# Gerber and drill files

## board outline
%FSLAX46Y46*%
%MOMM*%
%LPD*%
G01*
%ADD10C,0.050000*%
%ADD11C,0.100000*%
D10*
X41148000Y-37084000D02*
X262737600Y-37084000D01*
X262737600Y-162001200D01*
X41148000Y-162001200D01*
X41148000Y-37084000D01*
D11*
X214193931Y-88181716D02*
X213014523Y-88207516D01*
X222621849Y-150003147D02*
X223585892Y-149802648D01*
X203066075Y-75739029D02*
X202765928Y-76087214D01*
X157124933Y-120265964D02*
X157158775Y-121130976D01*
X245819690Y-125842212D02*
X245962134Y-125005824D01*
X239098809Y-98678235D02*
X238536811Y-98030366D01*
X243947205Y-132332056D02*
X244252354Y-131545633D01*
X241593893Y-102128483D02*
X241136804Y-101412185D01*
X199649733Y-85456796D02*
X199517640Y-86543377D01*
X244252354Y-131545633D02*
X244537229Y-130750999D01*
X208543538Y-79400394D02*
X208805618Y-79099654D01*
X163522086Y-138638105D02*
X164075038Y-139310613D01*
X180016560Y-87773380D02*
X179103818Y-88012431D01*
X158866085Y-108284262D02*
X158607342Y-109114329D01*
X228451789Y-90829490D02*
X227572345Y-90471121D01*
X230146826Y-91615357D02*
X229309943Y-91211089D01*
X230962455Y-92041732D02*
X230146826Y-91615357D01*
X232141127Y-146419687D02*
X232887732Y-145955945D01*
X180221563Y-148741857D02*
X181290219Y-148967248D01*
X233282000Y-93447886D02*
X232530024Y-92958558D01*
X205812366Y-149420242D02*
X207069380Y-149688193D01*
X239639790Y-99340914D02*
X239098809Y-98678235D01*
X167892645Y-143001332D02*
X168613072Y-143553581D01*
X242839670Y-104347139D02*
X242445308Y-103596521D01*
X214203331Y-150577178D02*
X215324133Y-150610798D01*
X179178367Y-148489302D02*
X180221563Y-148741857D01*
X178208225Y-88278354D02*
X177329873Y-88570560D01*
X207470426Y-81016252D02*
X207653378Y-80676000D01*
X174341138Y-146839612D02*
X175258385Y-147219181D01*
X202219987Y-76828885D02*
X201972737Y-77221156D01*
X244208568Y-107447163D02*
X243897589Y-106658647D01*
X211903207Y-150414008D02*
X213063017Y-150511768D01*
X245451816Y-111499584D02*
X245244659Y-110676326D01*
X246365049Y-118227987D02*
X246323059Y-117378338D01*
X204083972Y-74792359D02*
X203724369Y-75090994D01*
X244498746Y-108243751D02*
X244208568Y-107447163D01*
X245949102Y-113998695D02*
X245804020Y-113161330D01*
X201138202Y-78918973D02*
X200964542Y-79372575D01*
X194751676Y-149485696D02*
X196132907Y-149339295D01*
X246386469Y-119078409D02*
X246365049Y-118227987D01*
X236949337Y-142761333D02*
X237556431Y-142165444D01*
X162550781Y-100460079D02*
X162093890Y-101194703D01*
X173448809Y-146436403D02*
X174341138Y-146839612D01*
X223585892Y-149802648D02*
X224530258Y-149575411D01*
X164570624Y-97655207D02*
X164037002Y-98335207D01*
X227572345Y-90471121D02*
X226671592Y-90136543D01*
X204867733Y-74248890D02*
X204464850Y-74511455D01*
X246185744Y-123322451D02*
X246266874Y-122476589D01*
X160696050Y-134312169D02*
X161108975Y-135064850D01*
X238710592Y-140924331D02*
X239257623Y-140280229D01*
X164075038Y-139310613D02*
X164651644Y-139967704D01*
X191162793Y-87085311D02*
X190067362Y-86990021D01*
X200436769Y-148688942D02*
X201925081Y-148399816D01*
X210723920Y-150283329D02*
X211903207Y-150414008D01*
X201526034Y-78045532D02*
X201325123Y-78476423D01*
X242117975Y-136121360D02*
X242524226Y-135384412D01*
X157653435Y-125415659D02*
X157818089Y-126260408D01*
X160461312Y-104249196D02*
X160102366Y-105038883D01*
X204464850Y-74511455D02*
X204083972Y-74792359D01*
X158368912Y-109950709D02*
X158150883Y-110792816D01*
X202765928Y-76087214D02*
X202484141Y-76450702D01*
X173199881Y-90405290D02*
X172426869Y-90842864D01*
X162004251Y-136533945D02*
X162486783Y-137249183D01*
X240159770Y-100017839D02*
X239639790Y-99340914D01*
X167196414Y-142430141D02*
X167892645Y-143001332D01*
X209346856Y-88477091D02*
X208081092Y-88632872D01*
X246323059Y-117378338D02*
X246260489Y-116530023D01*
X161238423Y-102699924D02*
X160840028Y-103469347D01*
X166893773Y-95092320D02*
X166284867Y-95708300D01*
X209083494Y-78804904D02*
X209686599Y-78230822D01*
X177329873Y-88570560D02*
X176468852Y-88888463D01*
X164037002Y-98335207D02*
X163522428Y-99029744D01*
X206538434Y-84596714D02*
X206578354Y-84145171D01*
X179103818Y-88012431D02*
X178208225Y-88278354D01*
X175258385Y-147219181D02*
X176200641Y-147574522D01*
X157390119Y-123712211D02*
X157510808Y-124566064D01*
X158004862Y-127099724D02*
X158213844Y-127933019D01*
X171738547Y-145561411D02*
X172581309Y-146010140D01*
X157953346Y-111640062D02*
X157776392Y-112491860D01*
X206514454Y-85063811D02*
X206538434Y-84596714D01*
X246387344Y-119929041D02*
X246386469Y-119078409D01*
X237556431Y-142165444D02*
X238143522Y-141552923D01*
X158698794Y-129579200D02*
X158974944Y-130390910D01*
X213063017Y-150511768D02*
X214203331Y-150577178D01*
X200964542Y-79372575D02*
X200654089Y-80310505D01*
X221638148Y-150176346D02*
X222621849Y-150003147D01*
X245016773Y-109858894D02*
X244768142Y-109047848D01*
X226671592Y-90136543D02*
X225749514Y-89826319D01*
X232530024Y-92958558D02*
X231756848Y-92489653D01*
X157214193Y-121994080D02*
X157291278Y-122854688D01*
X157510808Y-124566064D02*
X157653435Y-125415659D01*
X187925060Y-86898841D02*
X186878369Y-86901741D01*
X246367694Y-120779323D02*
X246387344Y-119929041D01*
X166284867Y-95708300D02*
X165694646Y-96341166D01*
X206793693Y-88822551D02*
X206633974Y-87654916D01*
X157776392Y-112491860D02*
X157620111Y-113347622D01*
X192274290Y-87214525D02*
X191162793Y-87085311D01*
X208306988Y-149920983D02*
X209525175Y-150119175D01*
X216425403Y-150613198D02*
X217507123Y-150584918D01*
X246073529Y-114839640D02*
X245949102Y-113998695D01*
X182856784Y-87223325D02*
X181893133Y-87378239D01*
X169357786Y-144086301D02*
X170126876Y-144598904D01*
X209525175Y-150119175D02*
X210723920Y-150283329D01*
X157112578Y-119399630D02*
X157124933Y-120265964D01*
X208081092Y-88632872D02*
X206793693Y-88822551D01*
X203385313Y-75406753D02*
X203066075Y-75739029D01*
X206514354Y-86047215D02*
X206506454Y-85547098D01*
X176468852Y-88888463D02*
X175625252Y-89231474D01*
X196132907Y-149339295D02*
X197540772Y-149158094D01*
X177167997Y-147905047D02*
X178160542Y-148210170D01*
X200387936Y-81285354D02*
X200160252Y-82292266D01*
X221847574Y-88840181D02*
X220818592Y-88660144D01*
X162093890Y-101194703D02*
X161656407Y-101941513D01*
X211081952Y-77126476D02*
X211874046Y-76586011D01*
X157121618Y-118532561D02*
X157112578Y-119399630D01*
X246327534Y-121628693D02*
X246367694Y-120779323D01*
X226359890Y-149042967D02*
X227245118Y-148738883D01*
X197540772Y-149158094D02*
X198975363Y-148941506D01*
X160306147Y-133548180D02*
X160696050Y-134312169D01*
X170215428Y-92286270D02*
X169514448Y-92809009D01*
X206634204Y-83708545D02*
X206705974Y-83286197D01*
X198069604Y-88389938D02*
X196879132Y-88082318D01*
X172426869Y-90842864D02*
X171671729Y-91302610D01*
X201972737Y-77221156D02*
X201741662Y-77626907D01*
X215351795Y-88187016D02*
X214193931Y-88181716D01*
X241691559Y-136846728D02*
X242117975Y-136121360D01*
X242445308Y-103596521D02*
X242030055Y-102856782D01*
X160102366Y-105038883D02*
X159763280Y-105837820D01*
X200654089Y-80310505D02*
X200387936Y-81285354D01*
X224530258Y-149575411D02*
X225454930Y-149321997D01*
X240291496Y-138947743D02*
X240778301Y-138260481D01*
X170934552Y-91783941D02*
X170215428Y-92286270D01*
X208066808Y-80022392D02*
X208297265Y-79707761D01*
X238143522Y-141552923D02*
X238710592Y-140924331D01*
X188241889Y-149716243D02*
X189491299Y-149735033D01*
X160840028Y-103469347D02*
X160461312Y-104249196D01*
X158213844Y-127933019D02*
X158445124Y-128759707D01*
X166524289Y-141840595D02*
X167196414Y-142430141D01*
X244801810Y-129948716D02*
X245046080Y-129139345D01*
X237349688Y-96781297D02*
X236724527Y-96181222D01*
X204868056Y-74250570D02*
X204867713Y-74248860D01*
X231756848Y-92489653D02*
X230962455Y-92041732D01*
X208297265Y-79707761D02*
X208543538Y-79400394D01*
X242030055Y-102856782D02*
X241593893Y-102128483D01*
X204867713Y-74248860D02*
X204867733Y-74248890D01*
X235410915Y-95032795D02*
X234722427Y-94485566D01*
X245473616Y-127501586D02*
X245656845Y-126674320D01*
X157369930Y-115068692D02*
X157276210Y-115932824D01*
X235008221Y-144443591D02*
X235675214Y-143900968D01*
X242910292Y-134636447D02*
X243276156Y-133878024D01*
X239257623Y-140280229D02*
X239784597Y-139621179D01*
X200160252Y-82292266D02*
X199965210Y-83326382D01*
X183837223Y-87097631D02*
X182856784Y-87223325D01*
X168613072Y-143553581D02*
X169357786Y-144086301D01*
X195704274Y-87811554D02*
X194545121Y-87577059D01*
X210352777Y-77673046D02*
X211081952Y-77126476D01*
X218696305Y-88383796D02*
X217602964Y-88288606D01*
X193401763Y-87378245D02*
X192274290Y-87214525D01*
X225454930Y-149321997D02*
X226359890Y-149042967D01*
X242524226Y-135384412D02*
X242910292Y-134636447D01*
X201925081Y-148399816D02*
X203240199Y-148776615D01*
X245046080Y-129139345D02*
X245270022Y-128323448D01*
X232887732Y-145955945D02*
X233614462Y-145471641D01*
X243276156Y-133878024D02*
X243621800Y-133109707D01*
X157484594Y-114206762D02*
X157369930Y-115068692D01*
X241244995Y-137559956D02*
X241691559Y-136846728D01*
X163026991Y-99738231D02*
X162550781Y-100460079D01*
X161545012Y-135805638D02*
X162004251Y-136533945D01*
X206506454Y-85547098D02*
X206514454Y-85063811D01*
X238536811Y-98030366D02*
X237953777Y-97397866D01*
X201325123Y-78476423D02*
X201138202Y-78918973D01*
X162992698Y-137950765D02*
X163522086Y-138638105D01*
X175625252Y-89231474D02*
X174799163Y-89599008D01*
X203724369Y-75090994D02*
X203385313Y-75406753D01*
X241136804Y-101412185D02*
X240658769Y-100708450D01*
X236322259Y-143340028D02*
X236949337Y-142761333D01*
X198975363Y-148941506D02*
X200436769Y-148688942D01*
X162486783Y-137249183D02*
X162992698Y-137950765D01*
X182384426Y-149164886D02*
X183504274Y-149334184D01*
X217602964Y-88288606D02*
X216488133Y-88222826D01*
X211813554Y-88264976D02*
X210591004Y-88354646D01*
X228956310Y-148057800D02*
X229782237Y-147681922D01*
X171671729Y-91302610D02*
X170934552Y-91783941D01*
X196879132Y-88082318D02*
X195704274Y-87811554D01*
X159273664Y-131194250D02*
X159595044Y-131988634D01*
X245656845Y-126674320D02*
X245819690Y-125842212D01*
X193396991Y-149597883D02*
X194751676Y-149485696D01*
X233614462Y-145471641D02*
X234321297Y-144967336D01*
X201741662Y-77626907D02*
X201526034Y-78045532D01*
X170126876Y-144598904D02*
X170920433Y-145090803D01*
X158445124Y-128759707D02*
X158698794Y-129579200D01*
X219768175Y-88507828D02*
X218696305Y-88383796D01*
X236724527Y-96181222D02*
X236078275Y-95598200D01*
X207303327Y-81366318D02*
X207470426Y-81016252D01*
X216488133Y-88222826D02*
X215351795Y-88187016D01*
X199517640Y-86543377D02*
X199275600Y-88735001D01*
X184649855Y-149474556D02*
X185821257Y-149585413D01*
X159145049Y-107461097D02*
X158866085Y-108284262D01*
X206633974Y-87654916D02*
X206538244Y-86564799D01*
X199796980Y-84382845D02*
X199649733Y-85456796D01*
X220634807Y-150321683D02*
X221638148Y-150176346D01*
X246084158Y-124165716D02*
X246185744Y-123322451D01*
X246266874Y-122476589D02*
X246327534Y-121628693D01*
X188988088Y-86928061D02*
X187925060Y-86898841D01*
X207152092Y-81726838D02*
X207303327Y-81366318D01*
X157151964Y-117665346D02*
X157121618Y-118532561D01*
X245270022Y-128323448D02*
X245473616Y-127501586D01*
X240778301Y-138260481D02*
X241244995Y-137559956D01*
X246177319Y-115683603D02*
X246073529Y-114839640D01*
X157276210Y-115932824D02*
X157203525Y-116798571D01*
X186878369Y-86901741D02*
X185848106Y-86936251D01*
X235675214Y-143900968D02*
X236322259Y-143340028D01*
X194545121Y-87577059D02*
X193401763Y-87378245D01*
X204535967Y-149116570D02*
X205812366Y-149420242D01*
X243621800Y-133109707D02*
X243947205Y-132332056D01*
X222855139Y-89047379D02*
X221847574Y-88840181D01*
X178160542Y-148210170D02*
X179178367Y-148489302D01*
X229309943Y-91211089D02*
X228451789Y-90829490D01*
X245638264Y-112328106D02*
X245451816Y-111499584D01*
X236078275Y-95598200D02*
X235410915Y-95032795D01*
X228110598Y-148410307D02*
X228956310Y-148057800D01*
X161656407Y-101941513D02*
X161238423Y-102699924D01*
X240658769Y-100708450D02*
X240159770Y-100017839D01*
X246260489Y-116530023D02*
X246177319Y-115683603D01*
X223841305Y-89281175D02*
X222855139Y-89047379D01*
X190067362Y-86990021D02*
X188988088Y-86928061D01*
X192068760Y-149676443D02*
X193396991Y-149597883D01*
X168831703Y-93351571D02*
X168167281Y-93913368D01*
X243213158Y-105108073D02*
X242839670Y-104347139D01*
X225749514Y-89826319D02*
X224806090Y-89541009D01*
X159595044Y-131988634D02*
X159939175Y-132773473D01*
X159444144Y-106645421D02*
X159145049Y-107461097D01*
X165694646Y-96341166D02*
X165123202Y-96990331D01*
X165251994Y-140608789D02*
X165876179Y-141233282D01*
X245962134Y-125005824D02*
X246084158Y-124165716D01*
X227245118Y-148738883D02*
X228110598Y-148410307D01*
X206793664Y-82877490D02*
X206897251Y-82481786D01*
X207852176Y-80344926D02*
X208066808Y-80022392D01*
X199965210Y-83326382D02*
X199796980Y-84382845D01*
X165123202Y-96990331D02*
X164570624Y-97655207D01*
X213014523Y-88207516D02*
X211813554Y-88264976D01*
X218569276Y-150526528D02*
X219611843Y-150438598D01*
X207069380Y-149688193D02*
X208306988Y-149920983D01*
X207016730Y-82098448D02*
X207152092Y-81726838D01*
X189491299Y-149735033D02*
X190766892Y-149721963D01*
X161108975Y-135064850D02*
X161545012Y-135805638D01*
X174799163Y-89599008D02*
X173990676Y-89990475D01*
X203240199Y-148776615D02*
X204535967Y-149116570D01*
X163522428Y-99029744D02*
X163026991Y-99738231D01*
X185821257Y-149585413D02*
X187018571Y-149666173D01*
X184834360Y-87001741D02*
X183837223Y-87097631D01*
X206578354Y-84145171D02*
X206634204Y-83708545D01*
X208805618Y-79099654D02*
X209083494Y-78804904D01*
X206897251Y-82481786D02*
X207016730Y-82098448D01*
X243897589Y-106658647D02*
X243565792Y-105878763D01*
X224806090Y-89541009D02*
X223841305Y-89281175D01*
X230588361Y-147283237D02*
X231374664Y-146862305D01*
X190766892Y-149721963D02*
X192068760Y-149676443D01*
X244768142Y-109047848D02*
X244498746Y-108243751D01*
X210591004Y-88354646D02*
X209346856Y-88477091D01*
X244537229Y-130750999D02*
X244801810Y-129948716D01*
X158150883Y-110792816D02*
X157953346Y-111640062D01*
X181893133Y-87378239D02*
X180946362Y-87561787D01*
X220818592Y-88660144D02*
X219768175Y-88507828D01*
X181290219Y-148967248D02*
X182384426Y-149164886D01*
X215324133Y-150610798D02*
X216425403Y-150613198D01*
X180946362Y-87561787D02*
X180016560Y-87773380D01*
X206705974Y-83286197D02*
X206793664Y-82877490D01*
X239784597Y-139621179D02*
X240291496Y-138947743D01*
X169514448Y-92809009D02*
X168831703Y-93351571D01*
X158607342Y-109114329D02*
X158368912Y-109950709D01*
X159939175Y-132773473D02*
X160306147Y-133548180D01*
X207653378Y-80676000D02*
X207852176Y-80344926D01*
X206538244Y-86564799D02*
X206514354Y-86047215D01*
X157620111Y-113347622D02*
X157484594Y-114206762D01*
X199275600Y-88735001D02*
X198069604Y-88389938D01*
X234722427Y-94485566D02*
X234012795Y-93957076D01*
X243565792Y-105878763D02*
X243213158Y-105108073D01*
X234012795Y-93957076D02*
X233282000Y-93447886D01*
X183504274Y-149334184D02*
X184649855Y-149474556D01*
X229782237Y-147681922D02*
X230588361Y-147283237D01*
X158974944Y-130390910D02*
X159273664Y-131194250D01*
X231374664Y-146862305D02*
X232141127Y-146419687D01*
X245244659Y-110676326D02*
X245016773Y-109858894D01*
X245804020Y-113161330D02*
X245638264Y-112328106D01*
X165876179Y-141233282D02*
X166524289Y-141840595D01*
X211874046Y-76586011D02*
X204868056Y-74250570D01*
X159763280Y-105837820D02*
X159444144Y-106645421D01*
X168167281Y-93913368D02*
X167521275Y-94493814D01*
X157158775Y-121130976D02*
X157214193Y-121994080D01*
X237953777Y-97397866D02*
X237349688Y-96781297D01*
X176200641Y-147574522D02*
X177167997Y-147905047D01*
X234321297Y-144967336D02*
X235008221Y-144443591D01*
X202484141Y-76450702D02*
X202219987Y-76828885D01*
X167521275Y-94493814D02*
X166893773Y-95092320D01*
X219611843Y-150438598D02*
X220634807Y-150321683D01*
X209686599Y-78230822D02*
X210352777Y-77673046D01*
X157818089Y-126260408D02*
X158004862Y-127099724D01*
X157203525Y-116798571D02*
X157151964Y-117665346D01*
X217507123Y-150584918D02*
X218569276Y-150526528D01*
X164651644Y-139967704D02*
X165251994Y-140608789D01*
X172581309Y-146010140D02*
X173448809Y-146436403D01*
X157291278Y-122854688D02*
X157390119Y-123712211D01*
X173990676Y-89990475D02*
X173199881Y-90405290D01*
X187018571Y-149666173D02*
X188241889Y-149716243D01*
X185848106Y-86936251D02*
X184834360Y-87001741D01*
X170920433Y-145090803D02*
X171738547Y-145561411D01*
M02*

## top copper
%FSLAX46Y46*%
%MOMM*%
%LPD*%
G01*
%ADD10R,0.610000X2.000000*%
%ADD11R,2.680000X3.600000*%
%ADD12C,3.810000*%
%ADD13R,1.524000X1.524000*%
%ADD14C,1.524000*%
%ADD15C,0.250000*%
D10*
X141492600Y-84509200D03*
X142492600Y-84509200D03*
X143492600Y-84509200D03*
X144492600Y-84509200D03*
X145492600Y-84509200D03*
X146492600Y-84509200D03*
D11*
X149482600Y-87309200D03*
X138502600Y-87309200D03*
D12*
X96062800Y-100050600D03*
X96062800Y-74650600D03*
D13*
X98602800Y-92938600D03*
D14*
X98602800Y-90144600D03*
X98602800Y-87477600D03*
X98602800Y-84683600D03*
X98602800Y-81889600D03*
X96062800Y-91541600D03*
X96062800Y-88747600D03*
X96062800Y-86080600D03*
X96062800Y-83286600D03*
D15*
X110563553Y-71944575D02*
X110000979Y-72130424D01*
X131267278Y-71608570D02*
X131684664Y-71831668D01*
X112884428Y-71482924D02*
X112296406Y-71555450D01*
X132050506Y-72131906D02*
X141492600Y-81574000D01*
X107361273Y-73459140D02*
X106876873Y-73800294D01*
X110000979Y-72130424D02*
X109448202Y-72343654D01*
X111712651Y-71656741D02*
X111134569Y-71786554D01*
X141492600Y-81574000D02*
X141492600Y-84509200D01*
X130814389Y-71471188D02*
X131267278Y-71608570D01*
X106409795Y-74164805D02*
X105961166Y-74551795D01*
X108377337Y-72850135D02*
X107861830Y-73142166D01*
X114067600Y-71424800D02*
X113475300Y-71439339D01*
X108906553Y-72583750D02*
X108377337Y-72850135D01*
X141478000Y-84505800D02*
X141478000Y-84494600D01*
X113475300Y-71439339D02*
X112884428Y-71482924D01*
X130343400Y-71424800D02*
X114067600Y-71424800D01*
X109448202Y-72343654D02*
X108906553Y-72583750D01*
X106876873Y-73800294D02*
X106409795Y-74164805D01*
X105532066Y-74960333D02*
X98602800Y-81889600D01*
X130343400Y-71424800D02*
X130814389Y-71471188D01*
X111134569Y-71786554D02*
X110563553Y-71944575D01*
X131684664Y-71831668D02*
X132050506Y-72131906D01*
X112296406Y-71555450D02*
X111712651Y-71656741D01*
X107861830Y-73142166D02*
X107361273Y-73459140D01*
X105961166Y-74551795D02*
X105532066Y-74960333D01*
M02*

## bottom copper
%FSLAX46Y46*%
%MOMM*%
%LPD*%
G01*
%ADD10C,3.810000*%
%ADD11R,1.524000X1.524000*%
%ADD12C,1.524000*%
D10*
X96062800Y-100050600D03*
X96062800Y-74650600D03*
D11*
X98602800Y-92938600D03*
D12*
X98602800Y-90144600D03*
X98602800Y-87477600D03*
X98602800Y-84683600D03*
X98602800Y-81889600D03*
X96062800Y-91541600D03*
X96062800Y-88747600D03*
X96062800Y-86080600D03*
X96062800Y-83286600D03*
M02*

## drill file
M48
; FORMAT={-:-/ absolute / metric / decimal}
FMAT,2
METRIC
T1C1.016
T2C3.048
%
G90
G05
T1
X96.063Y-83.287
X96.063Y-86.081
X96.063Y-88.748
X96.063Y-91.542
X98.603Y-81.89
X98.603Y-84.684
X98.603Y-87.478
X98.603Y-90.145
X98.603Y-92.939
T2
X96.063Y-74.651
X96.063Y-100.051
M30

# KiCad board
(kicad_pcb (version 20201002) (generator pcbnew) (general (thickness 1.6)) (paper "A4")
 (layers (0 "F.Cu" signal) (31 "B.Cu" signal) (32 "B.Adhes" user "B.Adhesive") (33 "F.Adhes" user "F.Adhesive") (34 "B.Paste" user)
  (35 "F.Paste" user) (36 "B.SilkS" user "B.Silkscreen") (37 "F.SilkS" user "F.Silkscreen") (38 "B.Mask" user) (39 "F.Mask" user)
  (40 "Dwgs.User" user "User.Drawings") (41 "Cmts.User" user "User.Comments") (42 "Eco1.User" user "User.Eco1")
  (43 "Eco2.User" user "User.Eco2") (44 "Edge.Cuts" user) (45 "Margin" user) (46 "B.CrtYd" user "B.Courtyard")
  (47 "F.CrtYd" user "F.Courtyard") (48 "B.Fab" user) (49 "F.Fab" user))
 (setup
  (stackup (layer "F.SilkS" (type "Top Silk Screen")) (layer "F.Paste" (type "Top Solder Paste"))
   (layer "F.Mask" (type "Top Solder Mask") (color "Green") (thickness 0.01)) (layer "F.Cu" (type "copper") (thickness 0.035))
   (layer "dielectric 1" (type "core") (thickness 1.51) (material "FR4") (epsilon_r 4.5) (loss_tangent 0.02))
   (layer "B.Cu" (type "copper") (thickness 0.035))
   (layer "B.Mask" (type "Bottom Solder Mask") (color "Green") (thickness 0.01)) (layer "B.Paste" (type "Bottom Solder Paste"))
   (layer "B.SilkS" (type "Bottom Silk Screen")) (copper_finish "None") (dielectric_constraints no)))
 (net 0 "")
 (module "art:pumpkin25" (layer "F.Cu") (at 201.0156 117.475)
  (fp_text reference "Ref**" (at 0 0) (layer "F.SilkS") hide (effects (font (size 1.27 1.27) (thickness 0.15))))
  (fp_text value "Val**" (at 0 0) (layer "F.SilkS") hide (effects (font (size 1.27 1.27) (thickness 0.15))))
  (fp_line (start 13.178331 -29.293284) (end 11.998923 -29.267484) (layer "Edge.Cuts") (width 0.1))
  (fp_line (start 21.606249 32.528147) (end 22.570292 32.327648) (layer "Edge.Cuts") (width 0.1))
  (fp_line (start 2.050475 -41.735971) (end 1.750328 -41.387786) (layer "Edge.Cuts") (width 0.1))
  (fp_line (start -43.890667 2.790964) (end -43.856825 3.655976) (layer "Edge.Cuts") (width 0.1))
  (fp_line (start 44.80409 8.367212) (end 44.946534 7.530824) (layer "Edge.Cuts") (width 0.1))
  (fp_line (start 38.083209 -18.796765) (end 37.521211 -19.444634) (layer "Edge.Cuts") (width 0.1))
  (fp_line (start 42.931605 14.857056) (end 43.236754 14.070633) (layer "Edge.Cuts") (width 0.1))
  (fp_line (start 40.578293 -15.346517) (end 40.121204 -16.062815) (layer "Edge.Cuts") (width 0.1))
  (fp_line (start -1.365867 -32.018204) (end -1.49796 -30.931623) (layer "Edge.Cuts") (width 0.1))
  (fp_line (start 43.236754 14.070633) (end 43.521629 13.275999) (layer "Edge.Cuts") (width 0.1))
  (fp_line (start 7.527938 -38.074606) (end 7.790018 -38.375346) (layer "Edge.Cuts") (width 0.1))
  (fp_line (start -37.493514 21.163105) (end -36.940562 21.835613) (layer "Edge.Cuts") (width 0.1))
  (fp_line (start -20.99904 -29.70162) (end -21.911782 -29.462569) (layer "Edge.Cuts") (width 0.1))
  (fp_line (start -42.149515 -9.190738) (end -42.408258 -8.360671) (layer "Edge.Cuts") (width 0.1))
  (fp_line (start 27.436189 -26.64551) (end 26.556745 -27.003879) (layer "Edge.Cuts") (width 0.1))
  (fp_line (start 29.131226 -25.859643) (end 28.294343 -26.263911) (layer "Edge.Cuts") (width 0.1))
  (fp_line (start 29.946855 -25.433268) (end 29.131226 -25.859643) (layer "Edge.Cuts") (width 0.1))
  (fp_line (start 31.125527 28.944687) (end 31.872132 28.480945) (layer "Edge.Cuts") (width 0.1))
  (fp_line (start -20.794037 31.266857) (end -19.725381 31.492248) (layer "Edge.Cuts") (width 0.1))
  (fp_line (start 32.2664 -24.027114) (end 31.514424 -24.516442) (layer "Edge.Cuts") (width 0.1))
  (fp_line (start 4.796766 31.945242) (end 6.05378 32.213193) (layer "Edge.Cuts") (width 0.1))
  (fp_line (start 38.62419 -18.134086) (end 38.083209 -18.796765) (layer "Edge.Cuts") (width 0.1))
  (fp_line (start -33.122955 25.526332) (end -32.402528 26.078581) (layer "Edge.Cuts") (width 0.1))
  (fp_line (start 41.82407 -13.127861) (end 41.429708 -13.878479) (layer "Edge.Cuts") (width 0.1))
  (fp_line (start 13.187731 33.102178) (end 14.308533 33.135798) (layer "Edge.Cuts") (width 0.1))
  (fp_line (start -21.837233 31.014302) (end -20.794037 31.266857) (layer "Edge.Cuts") (width 0.1))
  (fp_line (start -22.807375 -29.196646) (end -23.685727 -28.90444) (layer "Edge.Cuts") (width 0.1))
  (fp_line (start 6.454826 -36.458748) (end 6.637778 -36.799) (layer "Edge.Cuts") (width 0.1))
  (fp_line (start -26.674462 29.364612) (end -25.757215 29.744181) (layer "Edge.Cuts") (width 0.1))
  (fp_line (start 1.204387 -40.646115) (end 0.957137 -40.253844) (layer "Edge.Cuts") (width 0.1))
  (fp_line (start 43.192968 -10.027837) (end 42.881989 -10.816353) (layer "Edge.Cuts") (width 0.1))
  (fp_line (start 10.887607 32.939008) (end 12.047417 33.036768) (layer "Edge.Cuts") (width 0.1))
  (fp_line (start 44.436216 -5.975416) (end 44.229059 -6.798674) (layer "Edge.Cuts") (width 0.1))
  (fp_line (start 45.349449 0.752987) (end 45.307459 -0.096662) (layer "Edge.Cuts") (width 0.1))
  (fp_line (start 3.068372 -42.682641) (end 2.708769 -42.384006) (layer "Edge.Cuts") (width 0.1))
  (fp_line (start 43.483146 -9.231249) (end 43.192968 -10.027837) (layer "Edge.Cuts") (width 0.1))
  (fp_line (start 44.933502 -3.476305) (end 44.78842 -4.31367) (layer "Edge.Cuts") (width 0.1))
  (fp_line (start 0.122602 -38.556027) (end -0.051058 -38.102425) (layer "Edge.Cuts") (width 0.1))
  (fp_line (start -6.263924 32.010696) (end -4.882693 31.864295) (layer "Edge.Cuts") (width 0.1))
  (fp_line (start 45.370869 1.603409) (end 45.349449 0.752987) (layer "Edge.Cuts") (width 0.1))
  (fp_line (start 35.933737 25.286333) (end 36.540831 24.690444) (layer "Edge.Cuts") (width 0.1))
  (fp_line (start -38.464819 -17.014921) (end -38.92171 -16.280297) (layer "Edge.Cuts") (width 0.1))
  (fp_line (start -27.566791 28.961403) (end -26.674462 29.364612) (layer "Edge.Cuts") (width 0.1))
  (fp_line (start 22.570292 32.327648) (end 23.514658 32.100411) (layer "Edge.Cuts") (width 0.1))
  (fp_line (start -36.444976 -19.819793) (end -36.978598 -19.139793) (layer "Edge.Cuts") (width 0.1))
  (fp_line (start 26.556745 -27.003879) (end 25.655992 -27.338457) (layer "Edge.Cuts") (width 0.1))
  (fp_line (start 3.852133 -43.22611) (end 3.44925 -42.963545) (layer "Edge.Cuts") (width 0.1))
  (fp_line (start 45.170144 5.847451) (end 45.251274 5.001589) (layer "Edge.Cuts") (width 0.1))
  (fp_line (start -40.31955 16.837169) (end -39.906625 17.58985) (layer "Edge.Cuts") (width 0.1))
  (fp_line (start 37.694992 23.449331) (end 38.242023 22.805229) (layer "Edge.Cuts") (width 0.1))
  (fp_line (start -36.940562 21.835613) (end -36.363956 22.492704) (layer "Edge.Cuts") (width 0.1))
  (fp_line (start -9.852807 -30.389689) (end -10.948238 -30.484979) (layer "Edge.Cuts") (width 0.1))
  (fp_line (start -0.578831 31.213942) (end 0.909481 30.924816) (layer "Edge.Cuts") (width 0.1))
  (fp_line (start 9.70832 32.808329) (end 10.887607 32.939008) (layer "Edge.Cuts") (width 0.1))
  (fp_line (start 0.510434 -39.429468) (end 0.309523 -38.998577) (layer "Edge.Cuts") (width 0.1))
  (fp_line (start 41.102375 18.64636) (end 41.508626 17.909412) (layer "Edge.Cuts") (width 0.1))
  (fp_line (start -43.362165 7.940659) (end -43.197511 8.785408) (layer "Edge.Cuts") (width 0.1))
  (fp_line (start -40.554288 -13.225804) (end -40.913234 -12.436117) (layer "Edge.Cuts") (width 0.1))
  (fp_line (start 3.44925 -42.963545) (end 3.068372 -42.682641) (layer "Edge.Cuts") (width 0.1))
  (fp_line (start -42.646688 -7.524291) (end -42.864717 -6.682184) (layer "Edge.Cuts") (width 0.1))
  (fp_line (start 1.750328 -41.387786) (end 1.468541 -41.024298) (layer "Edge.Cuts") (width 0.1))
  (fp_line (start -27.815719 -27.06971) (end -28.588731 -26.632136) (layer "Edge.Cuts") (width 0.1))
  (fp_line (start -39.011349 19.058945) (end -38.528817 19.774183) (layer "Edge.Cuts") (width 0.1))
  (fp_line (start 39.14417 -17.457161) (end 38.62419 -18.134086) (layer "Edge.Cuts") (width 0.1))
  (fp_line (start -33.819186 24.955141) (end -33.122955 25.526332) (layer "Edge.Cuts") (width 0.1))
  (fp_line (start 8.331256 -28.997909) (end 7.065492 -28.842128) (layer "Edge.Cuts") (width 0.1))
  (fp_line (start 45.307459 -0.096662) (end 45.244889 -0.944977) (layer "Edge.Cuts") (width 0.1))
  (fp_line (start -39.777177 -14.775076) (end -40.175572 -14.005653) (layer "Edge.Cuts") (width 0.1))
  (fp_line (start -34.121827 -22.38268) (end -34.730733 -21.7667) (layer "Edge.Cuts") (width 0.1))
  (fp_line (start 8.067894 -38.670096) (end 8.670999 -39.244178) (layer "Edge.Cuts") (width 0.1))
  (fp_line (start -23.685727 -28.90444) (end -24.546748 -28.586537) (layer "Edge.Cuts") (width 0.1))
  (fp_line (start -36.978598 -19.139793) (end -37.493172 -18.445256) (layer "Edge.Cuts") (width 0.1))
  (fp_line (start 5.522834 -32.878286) (end 5.562754 -33.329829) (layer "Edge.Cuts") (width 0.1))
  (fp_line (start -21.911782 -29.462569) (end -22.807375 -29.196646) (layer "Edge.Cuts") (width 0.1))
  (fp_line (start -25.757215 29.744181) (end -24.814959 30.099522) (layer "Edge.Cuts") (width 0.1))
  (fp_line (start -43.625481 6.237211) (end -43.504792 7.091064) (layer "Edge.Cuts") (width 0.1))
  (fp_line (start -43.010738 9.624724) (end -42.801756 10.458019) (layer "Edge.Cuts") (width 0.1))
  (fp_line (start -29.277053 28.086411) (end -28.434291 28.53514) (layer "Edge.Cuts") (width 0.1))
  (fp_line (start -43.062254 -5.834938) (end -43.239208 -4.98314) (layer "Edge.Cuts") (width 0.1))
  (fp_line (start 5.498854 -32.411189) (end 5.522834 -32.878286) (layer "Edge.Cuts") (width 0.1))
  (fp_line (start 45.371744 2.454041) (end 45.370869 1.603409) (layer "Edge.Cuts") (width 0.1))
  (fp_line (start 36.540831 24.690444) (end 37.127922 24.077923) (layer "Edge.Cuts") (width 0.1))
  (fp_line (start -42.316806 12.1042) (end -42.040656 12.91591) (layer "Edge.Cuts") (width 0.1))
  (fp_line (start 12.047417 33.036768) (end 13.187731 33.102178) (layer "Edge.Cuts") (width 0.1))
  (fp_line (start -0.051058 -38.102425) (end -0.361511 -37.164495) (layer "Edge.Cuts") (width 0.1))
  (fp_line (start 20.622548 32.701346) (end 21.606249 32.528147) (layer "Edge.Cuts") (width 0.1))
  (fp_line (start 44.001173 -7.616106) (end 43.752542 -8.427152) (layer "Edge.Cuts") (width 0.1))
  (fp_line (start 25.655992 -27.338457) (end 24.733914 -27.648681) (layer "Edge.Cuts") (width 0.1))
  (fp_line (start 31.514424 -24.516442) (end 30.741248 -24.985347) (layer "Edge.Cuts") (width 0.1))
  (fp_line (start -43.801407 4.51908) (end -43.724322 5.379688) (layer "Edge.Cuts") (width 0.1))
  (fp_line (start -43.504792 7.091064) (end -43.362165 7.940659) (layer "Edge.Cuts") (width 0.1))
  (fp_line (start -13.09054 -30.576159) (end -14.137231 -30.573259) (layer "Edge.Cuts") (width 0.1))
  (fp_line (start 45.352094 3.304323) (end 45.371744 2.454041) (layer "Edge.Cuts") (width 0.1))
  (fp_line (start -34.730733 -21.7667) (end -35.320954 -21.133834) (layer "Edge.Cuts") (width 0.1))
  (fp_line (start 5.778093 -28.652449) (end 5.618374 -29.820084) (layer "Edge.Cuts") (width 0.1))
  (fp_line (start -43.239208 -4.98314) (end -43.395489 -4.127378) (layer "Edge.Cuts") (width 0.1))
  (fp_line (start -8.74131 -30.260475) (end -9.852807 -30.389689) (layer "Edge.Cuts") (width 0.1))
  (fp_line (start 7.291388 32.445983) (end 8.509575 32.644175) (layer "Edge.Cuts") (width 0.1))
  (fp_line (start 15.409803 33.138198) (end 16.491523 33.109918) (layer "Edge.Cuts") (width 0.1))
  (fp_line (start 45.057929 -2.63536) (end 44.933502 -3.476305) (layer "Edge.Cuts") (width 0.1))
  (fp_line (start -18.158816 -30.251675) (end -19.122467 -30.096761) (layer "Edge.Cuts") (width 0.1))
  (fp_line (start -31.657814 26.611301) (end -30.888724 27.123904) (layer "Edge.Cuts") (width 0.1))
  (fp_line (start 8.509575 32.644175) (end 9.70832 32.808329) (layer "Edge.Cuts") (width 0.1))
  (fp_line (start -43.903022 1.92463) (end -43.890667 2.790964) (layer "Edge.Cuts") (width 0.1))
  (fp_line (start 7.065492 -28.842128) (end 5.778093 -28.652449) (layer "Edge.Cuts") (width 0.1))
  (fp_line (start 2.369713 -42.068247) (end 2.050475 -41.735971) (layer "Edge.Cuts") (width 0.1))
  (fp_line (start 5.498754 -31.427785) (end 5.490854 -31.927902) (layer "Edge.Cuts") (width 0.1))
  (fp_line (start -24.546748 -28.586537) (end -25.390348 -28.243526) (layer "Edge.Cuts") (width 0.1))
  (fp_line (start -4.882693 31.864295) (end -3.474828 31.683094) (layer "Edge.Cuts") (width 0.1))
  (fp_line (start -23.847603 30.430047) (end -22.855058 30.73517) (layer "Edge.Cuts") (width 0.1))
  (fp_line (start -0.627664 -36.189646) (end -0.855348 -35.182734) (layer "Edge.Cuts") (width 0.1))
  (fp_line (start 20.831974 -28.634819) (end 19.802992 -28.814856) (layer "Edge.Cuts") (width 0.1))
  (fp_line (start -38.92171 -16.280297) (end -39.359193 -15.533487) (layer "Edge.Cuts") (width 0.1))
  (fp_line (start 10.066352 -40.348524) (end 10.858446 -40.888989) (layer "Edge.Cuts") (width 0.1))
  (fp_line (start -43.893982 1.057561) (end -43.903022 1.92463) (layer "Edge.Cuts") (width 0.1))
  (fp_line (start 45.311934 4.153693) (end 45.352094 3.304323) (layer "Edge.Cuts") (width 0.1))
  (fp_line (start 25.34429 31.567967) (end 26.229518 31.263883) (layer "Edge.Cuts") (width 0.1))
  (fp_line (start -3.474828 31.683094) (end -2.040237 31.466506) (layer "Edge.Cuts") (width 0.1))
  (fp_line (start -40.709453 16.07318) (end -40.31955 16.837169) (layer "Edge.Cuts") (width 0.1))
  (fp_line (start -30.800172 -25.18873) (end -31.501152 -24.665991) (layer "Edge.Cuts") (width 0.1))
  (fp_line (start 5.618604 -33.766455) (end 5.690374 -34.188803) (layer "Edge.Cuts") (width 0.1))
  (fp_line (start -2.945996 -29.085062) (end -4.136468 -29.392682) (layer "Edge.Cuts") (width 0.1))
  (fp_line (start -28.588731 -26.632136) (end -29.343871 -26.17239) (layer "Edge.Cuts") (width 0.1))
  (fp_line (start 0.957137 -40.253844) (end 0.726062 -39.848093) (layer "Edge.Cuts") (width 0.1))
  (fp_line (start 14.336195 -29.287984) (end 13.178331 -29.293284) (layer "Edge.Cuts") (width 0.1))
  (fp_line (start 40.675959 19.371728) (end 41.102375 18.64636) (layer "Edge.Cuts") (width 0.1))
  (fp_line (start 41.429708 -13.878479) (end 41.014455 -14.618218) (layer "Edge.Cuts") (width 0.1))
  (fp_line (start -40.913234 -12.436117) (end -41.25232 -11.63718) (layer "Edge.Cuts") (width 0.1))
  (fp_line (start -0.361511 -37.164495) (end -0.627664 -36.189646) (layer "Edge.Cuts") (width 0.1))
  (fp_line (start 23.514658 32.100411) (end 24.43933 31.846997) (layer "Edge.Cuts") (width 0.1))
  (fp_line (start 39.275896 21.472743) (end 39.762701 20.785481) (layer "Edge.Cuts") (width 0.1))
  (fp_line (start -30.081048 -25.691059) (end -30.800172 -25.18873) (layer "Edge.Cuts") (width 0.1))
  (fp_line (start 7.051208 -37.452608) (end 7.281665 -37.767239) (layer "Edge.Cuts") (width 0.1))
  (fp_line (start 37.127922 24.077923) (end 37.694992 23.449331) (layer "Edge.Cuts") (width 0.1))
  (fp_line (start -12.773711 32.241243) (end -11.524301 32.260033) (layer "Edge.Cuts") (width 0.1))
  (fp_line (start -40.175572 -14.005653) (end -40.554288 -13.225804) (layer "Edge.Cuts") (width 0.1))
  (fp_line (start -42.801756 10.458019) (end -42.570476 11.284707) (layer "Edge.Cuts") (width 0.1))
  (fp_line (start -34.491311 24.365595) (end -33.819186 24.955141) (layer "Edge.Cuts") (width 0.1))
  (fp_line (start 43.78621 12.473716) (end 44.03048 11.664345) (layer "Edge.Cuts") (width 0.1))
  (fp_line (start 36.334088 -20.693703) (end 35.708927 -21.293778) (layer "Edge.Cuts") (width 0.1))
  (fp_line (start 3.852456 -43.22443) (end 3.852113 -43.22614) (layer "Edge.Cuts") (width 0.1))
  (fp_line (start 30.741248 -24.985347) (end 29.946855 -25.433268) (layer "Edge.Cuts") (width 0.1))
  (fp_line (start 7.281665 -37.767239) (end 7.527938 -38.074606) (layer "Edge.Cuts") (width 0.1))
  (fp_line (start 41.014455 -14.618218) (end 40.578293 -15.346517) (layer "Edge.Cuts") (width 0.1))
  (fp_line (start 3.852113 -43.22614) (end 3.852133 -43.22611) (layer "Edge.Cuts") (width 0.1))
  (fp_line (start 34.395315 -22.442205) (end 33.706827 -22.989434) (layer "Edge.Cuts") (width 0.1))
  (fp_line (start 44.458016 10.026586) (end 44.641245 9.19932) (layer "Edge.Cuts") (width 0.1))
  (fp_line (start -43.64567 -2.406308) (end -43.73939 -1.542176) (layer "Edge.Cuts") (width 0.1))
  (fp_line (start 33.992621 26.968591) (end 34.659614 26.425968) (layer "Edge.Cuts") (width 0.1))
  (fp_line (start 41.894692 17.161447) (end 42.260556 16.403024) (layer "Edge.Cuts") (width 0.1))
  (fp_line (start 38.242023 22.805229) (end 38.768997 22.146179) (layer "Edge.Cuts") (width 0.1))
  (fp_line (start -0.855348 -35.182734) (end -1.05039 -34.148618) (layer "Edge.Cuts") (width 0.1))
  (fp_line (start -17.178377 -30.377369) (end -18.158816 -30.251675) (layer "Edge.Cuts") (width 0.1))
  (fp_line (start -32.402528 26.078581) (end -31.657814 26.611301) (layer "Edge.Cuts") (width 0.1))
  (fp_line (start -5.311326 -29.663446) (end -6.470479 -29.897941) (layer "Edge.Cuts") (width 0.1))
  (fp_line (start 9.337177 -39.801954) (end 10.066352 -40.348524) (layer "Edge.Cuts") (width 0.1))
  (fp_line (start 17.680705 -29.091204) (end 16.587364 -29.186394) (layer "Edge.Cuts") (width 0.1))
  (fp_line (start -7.613837 -30.096755) (end -8.74131 -30.260475) (layer "Edge.Cuts") (width 0.1))
  (fp_line (start 24.43933 31.846997) (end 25.34429 31.567967) (layer "Edge.Cuts") (width 0.1))
  (fp_line (start 41.508626 17.909412) (end 41.894692 17.161447) (layer "Edge.Cuts") (width 0.1))
  (fp_line (start 0.909481 30.924816) (end 2.224599 31.301615) (layer "Edge.Cuts") (width 0.1))
  (fp_line (start 44.03048 11.664345) (end 44.254422 10.848448) (layer "Edge.Cuts") (width 0.1))
  (fp_line (start 31.872132 28.480945) (end 32.598862 27.996641) (layer "Edge.Cuts") (width 0.1))
  (fp_line (start 42.260556 16.403024) (end 42.6062 15.634707) (layer "Edge.Cuts") (width 0.1))
  (fp_line (start -43.531006 -3.268238) (end -43.64567 -2.406308) (layer "Edge.Cuts") (width 0.1))
  (fp_line (start 40.229395 20.084956) (end 40.675959 19.371728) (layer "Edge.Cuts") (width 0.1))
  (fp_line (start -37.988609 -17.736769) (end -38.464819 -17.014921) (layer "Edge.Cuts") (width 0.1))
  (fp_line (start -39.470588 18.330638) (end -39.011349 19.058945) (layer "Edge.Cuts") (width 0.1))
  (fp_line (start 5.490854 -31.927902) (end 5.498854 -32.411189) (layer "Edge.Cuts") (width 0.1))
  (fp_line (start 37.521211 -19.444634) (end 36.938177 -20.077134) (layer "Edge.Cuts") (width 0.1))
  (fp_line (start 0.309523 -38.998577) (end 0.122602 -38.556027) (layer "Edge.Cuts") (width 0.1))
  (fp_line (start -38.022902 20.475765) (end -37.493514 21.163105) (layer "Edge.Cuts") (width 0.1))
  (fp_line (start -25.390348 -28.243526) (end -26.216437 -27.875992) (layer "Edge.Cuts") (width 0.1))
  (fp_line (start 2.708769 -42.384006) (end 2.369713 -42.068247) (layer "Edge.Cuts") (width 0.1))
  (fp_line (start 40.121204 -16.062815) (end 39.643169 -16.76655) (layer "Edge.Cuts") (width 0.1))
  (fp_line (start 35.306659 25.865028) (end 35.933737 25.286333) (layer "Edge.Cuts") (width 0.1))
  (fp_line (start -2.040237 31.466506) (end -0.578831 31.213942) (layer "Edge.Cuts") (width 0.1))
  (fp_line (start -38.528817 19.774183) (end -38.022902 20.475765) (layer "Edge.Cuts") (width 0.1))
  (fp_line (start -18.631174 31.689886) (end -17.511326 31.859184) (layer "Edge.Cuts") (width 0.1))
  (fp_line (start 16.587364 -29.186394) (end 15.472533 -29.252174) (layer "Edge.Cuts") (width 0.1))
  (fp_line (start 10.797954 -29.210024) (end 9.575404 -29.120354) (layer "Edge.Cuts") (width 0.1))
  (fp_line (start 27.94071 30.5828) (end 28.766637 30.206922) (layer "Edge.Cuts") (width 0.1))
  (fp_line (start -29.343871 -26.17239) (end -30.081048 -25.691059) (layer "Edge.Cuts") (width 0.1))
  (fp_line (start -4.136468 -29.392682) (end -5.311326 -29.663446) (layer "Edge.Cuts") (width 0.1))
  (fp_line (start -41.741936 13.71925) (end -41.420556 14.513634) (layer "Edge.Cuts") (width 0.1))
  (fp_line (start 44.641245 9.19932) (end 44.80409 8.367212) (layer "Edge.Cuts") (width 0.1))
  (fp_line (start -7.618609 32.122883) (end -6.263924 32.010696) (layer "Edge.Cuts") (width 0.1))
  (fp_line (start 32.598862 27.996641) (end 33.305697 27.492336) (layer "Edge.Cuts") (width 0.1))
  (fp_line (start 0.726062 -39.848093) (end 0.510434 -39.429468) (layer "Edge.Cuts") (width 0.1))
  (fp_line (start -30.888724 27.123904) (end -30.095167 27.615803) (layer "Edge.Cuts") (width 0.1))
  (fp_line (start -42.570476 11.284707) (end -42.316806 12.1042) (layer "Edge.Cuts") (width 0.1))
  (fp_line (start 18.752575 -28.967172) (end 17.680705 -29.091204) (layer "Edge.Cuts") (width 0.1))
  (fp_line (start 35.708927 -21.293778) (end 35.062675 -21.8768) (layer "Edge.Cuts") (width 0.1))
  (fp_line (start 6.287727 -36.108682) (end 6.454826 -36.458748) (layer "Edge.Cuts") (width 0.1))
  (fp_line (start 15.472533 -29.252174) (end 14.336195 -29.287984) (layer "Edge.Cuts") (width 0.1))
  (fp_line (start -1.49796 -30.931623) (end -1.74 -28.739999) (layer "Edge.Cuts") (width 0.1))
  (fp_line (start -16.365745 31.999556) (end -15.194343 32.110413) (layer "Edge.Cuts") (width 0.1))
  (fp_line (start -41.870551 -10.013903) (end -42.149515 -9.190738) (layer "Edge.Cuts") (width 0.1))
  (fp_line (start 5.618374 -29.820084) (end 5.522644 -30.910201) (layer "Edge.Cuts") (width 0.1))
  (fp_line (start -1.21862 -33.092155) (end -1.365867 -32.018204) (layer "Edge.Cuts") (width 0.1))
  (fp_line (start 19.619207 32.846683) (end 20.622548 32.701346) (layer "Edge.Cuts") (width 0.1))
  (fp_line (start 45.068558 6.690716) (end 45.170144 5.847451) (layer "Edge.Cuts") (width 0.1))
  (fp_line (start 45.251274 5.001589) (end 45.311934 4.153693) (layer "Edge.Cuts") (width 0.1))
  (fp_line (start -12.027512 -30.546939) (end -13.09054 -30.576159) (layer "Edge.Cuts") (width 0.1))
  (fp_line (start 6.136492 -35.748162) (end 6.287727 -36.108682) (layer "Edge.Cuts") (width 0.1))
  (fp_line (start -43.863636 0.190346) (end -43.893982 1.057561) (layer "Edge.Cuts") (width 0.1))
  (fp_line (start 44.254422 10.848448) (end 44.458016 10.026586) (layer "Edge.Cuts") (width 0.1))
  (fp_line (start 39.762701 20.785481) (end 40.229395 20.084956) (layer "Edge.Cuts") (width 0.1))
  (fp_line (start 45.161719 -1.791397) (end 45.057929 -2.63536) (layer "Edge.Cuts") (width 0.1))
  (fp_line (start -43.73939 -1.542176) (end -43.812075 -0.676429) (layer "Edge.Cuts") (width 0.1))
  (fp_line (start -14.137231 -30.573259) (end -15.167494 -30.538749) (layer "Edge.Cuts") (width 0.1))
  (fp_line (start 34.659614 26.425968) (end 35.306659 25.865028) (layer "Edge.Cuts") (width 0.1))
  (fp_line (start -6.470479 -29.897941) (end -7.613837 -30.096755) (layer "Edge.Cuts") (width 0.1))
  (fp_line (start 3.520367 31.64157) (end 4.796766 31.945242) (layer "Edge.Cuts") (width 0.1))
  (fp_line (start 42.6062 15.634707) (end 42.931605 14.857056) (layer "Edge.Cuts") (width 0.1))
  (fp_line (start 21.839539 -28.427621) (end 20.831974 -28.634819) (layer "Edge.Cuts") (width 0.1))
  (fp_line (start -22.855058 30.73517) (end -21.837233 31.014302) (layer "Edge.Cuts") (width 0.1))
  (fp_line (start 28.294343 -26.263911) (end 27.436189 -26.64551) (layer "Edge.Cuts") (width 0.1))
  (fp_line (start 44.622664 -5.146894) (end 44.436216 -5.975416) (layer "Edge.Cuts") (width 0.1))
  (fp_line (start 35.062675 -21.8768) (end 34.395315 -22.442205) (layer "Edge.Cuts") (width 0.1))
  (fp_line (start 27.094998 30.935307) (end 27.94071 30.5828) (layer "Edge.Cuts") (width 0.1))
  (fp_line (start -39.359193 -15.533487) (end -39.777177 -14.775076) (layer "Edge.Cuts") (width 0.1))
  (fp_line (start 39.643169 -16.76655) (end 39.14417 -17.457161) (layer "Edge.Cuts") (width 0.1))
  (fp_line (start 45.244889 -0.944977) (end 45.161719 -1.791397) (layer "Edge.Cuts") (width 0.1))
  (fp_line (start 22.825705 -28.193825) (end 21.839539 -28.427621) (layer "Edge.Cuts") (width 0.1))
  (fp_line (start -10.948238 -30.484979) (end -12.027512 -30.546939) (layer "Edge.Cuts") (width 0.1))
  (fp_line (start -8.94684 32.201443) (end -7.618609 32.122883) (layer "Edge.Cuts") (width 0.1))
  (fp_line (start -32.183897 -24.123429) (end -32.848319 -23.561632) (layer "Edge.Cuts") (width 0.1))
  (fp_line (start 42.197558 -12.366927) (end 41.82407 -13.127861) (layer "Edge.Cuts") (width 0.1))
  (fp_line (start 24.733914 -27.648681) (end 23.79049 -27.933991) (layer "Edge.Cuts") (width 0.1))
  (fp_line (start -41.420556 14.513634) (end -41.076425 15.298473) (layer "Edge.Cuts") (width 0.1))
  (fp_line (start -41.571456 -10.829579) (end -41.870551 -10.013903) (layer "Edge.Cuts") (width 0.1))
  (fp_line (start -35.320954 -21.133834) (end -35.892398 -20.484669) (layer "Edge.Cuts") (width 0.1))
  (fp_line (start -35.763606 23.133789) (end -35.139421 23.758282) (layer "Edge.Cuts") (width 0.1))
  (fp_line (start 44.946534 7.530824) (end 45.068558 6.690716) (layer "Edge.Cuts") (width 0.1))
  (fp_line (start 26.229518 31.263883) (end 27.094998 30.935307) (layer "Edge.Cuts") (width 0.1))
  (fp_line (start 5.778064 -34.59751) (end 5.881651 -34.993214) (layer "Edge.Cuts") (width 0.1))
  (fp_line (start 6.836576 -37.130074) (end 7.051208 -37.452608) (layer "Edge.Cuts") (width 0.1))
  (fp_line (start -1.05039 -34.148618) (end -1.21862 -33.092155) (layer "Edge.Cuts") (width 0.1))
  (fp_line (start -35.892398 -20.484669) (end -36.444976 -19.819793) (layer "Edge.Cuts") (width 0.1))
  (fp_line (start 11.998923 -29.267484) (end 10.797954 -29.210024) (layer "Edge.Cuts") (width 0.1))
  (fp_line (start 17.553676 33.051528) (end 18.596243 32.963598) (layer "Edge.Cuts") (width 0.1))
  (fp_line (start 6.05378 32.213193) (end 7.291388 32.445983) (layer "Edge.Cuts") (width 0.1))
  (fp_line (start 6.00113 -35.376552) (end 6.136492 -35.748162) (layer "Edge.Cuts") (width 0.1))
  (fp_line (start -11.524301 32.260033) (end -10.248708 32.246963) (layer "Edge.Cuts") (width 0.1))
  (fp_line (start -39.906625 17.58985) (end -39.470588 18.330638) (layer "Edge.Cuts") (width 0.1))
  (fp_line (start -26.216437 -27.875992) (end -27.024924 -27.484525) (layer "Edge.Cuts") (width 0.1))
  (fp_line (start 2.224599 31.301615) (end 3.520367 31.64157) (layer "Edge.Cuts") (width 0.1))
  (fp_line (start -37.493172 -18.445256) (end -37.988609 -17.736769) (layer "Edge.Cuts") (width 0.1))
  (fp_line (start -15.194343 32.110413) (end -13.997029 32.191173) (layer "Edge.Cuts") (width 0.1))
  (fp_line (start -16.18124 -30.473259) (end -17.178377 -30.377369) (layer "Edge.Cuts") (width 0.1))
  (fp_line (start 5.562754 -33.329829) (end 5.618604 -33.766455) (layer "Edge.Cuts") (width 0.1))
  (fp_line (start 7.790018 -38.375346) (end 8.067894 -38.670096) (layer "Edge.Cuts") (width 0.1))
  (fp_line (start 5.881651 -34.993214) (end 6.00113 -35.376552) (layer "Edge.Cuts") (width 0.1))
  (fp_line (start 42.881989 -10.816353) (end 42.550192 -11.596237) (layer "Edge.Cuts") (width 0.1))
  (fp_line (start 23.79049 -27.933991) (end 22.825705 -28.193825) (layer "Edge.Cuts") (width 0.1))
  (fp_line (start 29.572761 29.808237) (end 30.359064 29.387305) (layer "Edge.Cuts") (width 0.1))
  (fp_line (start -10.248708 32.246963) (end -8.94684 32.201443) (layer "Edge.Cuts") (width 0.1))
  (fp_line (start 43.752542 -8.427152) (end 43.483146 -9.231249) (layer "Edge.Cuts") (width 0.1))
  (fp_line (start 9.575404 -29.120354) (end 8.331256 -28.997909) (layer "Edge.Cuts") (width 0.1))
  (fp_line (start 43.521629 13.275999) (end 43.78621 12.473716) (layer "Edge.Cuts") (width 0.1))
  (fp_line (start -42.864717 -6.682184) (end -43.062254 -5.834938) (layer "Edge.Cuts") (width 0.1))
  (fp_line (start -19.122467 -30.096761) (end -20.069238 -29.913213) (layer "Edge.Cuts") (width 0.1))
  (fp_line (start 19.802992 -28.814856) (end 18.752575 -28.967172) (layer "Edge.Cuts") (width 0.1))
  (fp_line (start -19.725381 31.492248) (end -18.631174 31.689886) (layer "Edge.Cuts") (width 0.1))
  (fp_line (start 14.308533 33.135798) (end 15.409803 33.138198) (layer "Edge.Cuts") (width 0.1))
  (fp_line (start -20.069238 -29.913213) (end -20.99904 -29.70162) (layer "Edge.Cuts") (width 0.1))
  (fp_line (start 5.690374 -34.188803) (end 5.778064 -34.59751) (layer "Edge.Cuts") (width 0.1))
  (fp_line (start 38.768997 22.146179) (end 39.275896 21.472743) (layer "Edge.Cuts") (width 0.1))
  (fp_line (start -31.501152 -24.665991) (end -32.183897 -24.123429) (layer "Edge.Cuts") (width 0.1))
  (fp_line (start -42.408258 -8.360671) (end -42.646688 -7.524291) (layer "Edge.Cuts") (width 0.1))
  (fp_line (start -41.076425 15.298473) (end -40.709453 16.07318) (layer "Edge.Cuts") (width 0.1))
  (fp_line (start 6.637778 -36.799) (end 6.836576 -37.130074) (layer "Edge.Cuts") (width 0.1))
  (fp_line (start 5.522644 -30.910201) (end 5.498754 -31.427785) (layer "Edge.Cuts") (width 0.1))
  (fp_line (start -43.395489 -4.127378) (end -43.531006 -3.268238) (layer "Edge.Cuts") (width 0.1))
  (fp_line (start -1.74 -28.739999) (end -2.945996 -29.085062) (layer "Edge.Cuts") (width 0.1))
  (fp_line (start 33.706827 -22.989434) (end 32.997195 -23.517924) (layer "Edge.Cuts") (width 0.1))
  (fp_line (start 42.550192 -11.596237) (end 42.197558 -12.366927) (layer "Edge.Cuts") (width 0.1))
  (fp_line (start 32.997195 -23.517924) (end 32.2664 -24.027114) (layer "Edge.Cuts") (width 0.1))
  (fp_line (start -17.511326 31.859184) (end -16.365745 31.999556) (layer "Edge.Cuts") (width 0.1))
  (fp_line (start 28.766637 30.206922) (end 29.572761 29.808237) (layer "Edge.Cuts") (width 0.1))
  (fp_line (start -42.040656 12.91591) (end -41.741936 13.71925) (layer "Edge.Cuts") (width 0.1))
  (fp_line (start 30.359064 29.387305) (end 31.125527 28.944687) (layer "Edge.Cuts") (width 0.1))
  (fp_line (start 44.229059 -6.798674) (end 44.001173 -7.616106) (layer "Edge.Cuts") (width 0.1))
  (fp_line (start 44.78842 -4.31367) (end 44.622664 -5.146894) (layer "Edge.Cuts") (width 0.1))
  (fp_line (start -35.139421 23.758282) (end -34.491311 24.365595) (layer "Edge.Cuts") (width 0.1))
  (fp_line (start 10.858446 -40.888989) (end 3.852456 -43.22443) (layer "Edge.Cuts") (width 0.1))
  (fp_line (start -41.25232 -11.63718) (end -41.571456 -10.829579) (layer "Edge.Cuts") (width 0.1))
  (fp_line (start -32.848319 -23.561632) (end -33.494325 -22.981186) (layer "Edge.Cuts") (width 0.1))
  (fp_line (start -43.856825 3.655976) (end -43.801407 4.51908) (layer "Edge.Cuts") (width 0.1))
  (fp_line (start 36.938177 -20.077134) (end 36.334088 -20.693703) (layer "Edge.Cuts") (width 0.1))
  (fp_line (start -24.814959 30.099522) (end -23.847603 30.430047) (layer "Edge.Cuts") (width 0.1))
  (fp_line (start 33.305697 27.492336) (end 33.992621 26.968591) (layer "Edge.Cuts") (width 0.1))
  (fp_line (start 1.468541 -41.024298) (end 1.204387 -40.646115) (layer "Edge.Cuts") (width 0.1))
  (fp_line (start -33.494325 -22.981186) (end -34.121827 -22.38268) (layer "Edge.Cuts") (width 0.1))
  (fp_line (start 18.596243 32.963598) (end 19.619207 32.846683) (layer "Edge.Cuts") (width 0.1))
  (fp_line (start 8.670999 -39.244178) (end 9.337177 -39.801954) (layer "Edge.Cuts") (width 0.1))
  (fp_line (start -43.197511 8.785408) (end -43.010738 9.624724) (layer "Edge.Cuts") (width 0.1))
  (fp_line (start -43.812075 -0.676429) (end -43.863636 0.190346) (layer "Edge.Cuts") (width 0.1))
  (fp_line (start 16.491523 33.109918) (end 17.553676 33.051528) (layer "Edge.Cuts") (width 0.1))
  (fp_line (start -36.363956 22.492704) (end -35.763606 23.133789) (layer "Edge.Cuts") (width 0.1))
  (fp_line (start -28.434291 28.53514) (end -27.566791 28.961403) (layer "Edge.Cuts") (width 0.1))
  (fp_line (start -43.724322 5.379688) (end -43.625481 6.237211) (layer "Edge.Cuts") (width 0.1))
  (fp_line (start -27.024924 -27.484525) (end -27.815719 -27.06971) (layer "Edge.Cuts") (width 0.1))
  (fp_line (start -13.997029 32.191173) (end -12.773711 32.241243) (layer "Edge.Cuts") (width 0.1))
  (fp_line (start -15.167494 -30.538749) (end -16.18124 -30.473259) (layer "Edge.Cuts") (width 0.1))
  (fp_line (start -30.095167 27.615803) (end -29.277053 28.086411) (layer "Edge.Cuts") (width 0.1)))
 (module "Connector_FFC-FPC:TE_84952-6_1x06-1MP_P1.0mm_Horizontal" (layer "F.Cu") (at 143.9926 86.3092)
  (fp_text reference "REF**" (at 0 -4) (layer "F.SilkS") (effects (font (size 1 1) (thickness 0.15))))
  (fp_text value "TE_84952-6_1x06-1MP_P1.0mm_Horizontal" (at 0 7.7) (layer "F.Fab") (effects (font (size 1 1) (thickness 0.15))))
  (pad "1" smd rect (at -2.5 -1.8) (size 0.61 2) (layers "F.Cu" "F.Paste" "F.Mask"))
  (pad "2" smd rect (at -1.5 -1.8) (size 0.61 2) (layers "F.Cu" "F.Paste" "F.Mask"))
  (pad "3" smd rect (at -0.5 -1.8) (size 0.61 2) (layers "F.Cu" "F.Paste" "F.Mask"))
  (pad "4" smd rect (at 0.5 -1.8) (size 0.61 2) (layers "F.Cu" "F.Paste" "F.Mask"))
  (pad "5" smd rect (at 1.5 -1.8) (size 0.61 2) (layers "F.Cu" "F.Paste" "F.Mask"))
  (pad "6" smd rect (at 2.5 -1.8) (size 0.61 2) (layers "F.Cu" "F.Paste" "F.Mask"))
  (pad "MP" smd rect (at 5.49 1) (size 2.68 3.6) (layers "F.Cu" "F.Paste" "F.Mask"))
  (pad "MP" smd rect (at -5.49 1) (size 2.68 3.6) (layers "F.Cu" "F.Paste" "F.Mask")))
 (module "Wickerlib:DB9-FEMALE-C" (layer "F.Cu") (at 97.3328 87.4776 90)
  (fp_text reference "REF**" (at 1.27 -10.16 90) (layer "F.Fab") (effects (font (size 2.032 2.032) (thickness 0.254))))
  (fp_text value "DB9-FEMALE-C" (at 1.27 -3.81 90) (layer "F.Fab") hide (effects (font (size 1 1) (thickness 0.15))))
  (pad "" thru_hole circle (at -12.573 -1.27 90) (size 3.81 3.81) (drill 3.048) (layers *.Cu *.Mask "F.SilkS"))
  (pad "" thru_hole circle (at 12.827 -1.27 90) (size 3.81 3.81) (drill 3.048) (layers *.Cu *.Mask "F.SilkS"))
  (pad "1" thru_hole rect (at -5.461 1.27 90) (size 1.524 1.524) (drill 1.016) (layers *.Cu *.Mask "F.SilkS"))
  (pad "2" thru_hole circle (at -2.667 1.27 90) (size 1.524 1.524) (drill 1.016) (layers *.Cu *.Mask "F.SilkS"))
  (pad "3" thru_hole circle (at 0 1.27 90) (size 1.524 1.524) (drill 1.016) (layers *.Cu *.Mask "F.SilkS"))
  (pad "4" thru_hole circle (at 2.794 1.27 90) (size 1.524 1.524) (drill 1.016) (layers *.Cu *.Mask "F.SilkS"))
  (pad "5" thru_hole circle (at 5.588 1.27 90) (size 1.524 1.524) (drill 1.016) (layers *.Cu *.Mask "F.SilkS"))
  (pad "6" thru_hole circle (at -4.064 -1.27 90) (size 1.524 1.524) (drill 1.016) (layers *.Cu *.Mask "F.SilkS"))
  (pad "7" thru_hole circle (at -1.27 -1.27 90) (size 1.524 1.524) (drill 1.016) (layers *.Cu *.Mask "F.SilkS"))
  (pad "8" thru_hole circle (at 1.397 -1.27 90) (size 1.524 1.524) (drill 1.016) (layers *.Cu *.Mask "F.SilkS"))
  (pad "9" thru_hole circle (at 4.191 -1.27 90) (size 1.524 1.524) (drill 1.016) (layers *.Cu *.Mask "F.SilkS")))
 (gr_rect (start 41.148 37.084) (end 262.7376 162.0012) (layer "Edge.Cuts") (width 0.05))
 (segment (start 110.563553 71.944575) (end 110.000979 72.130424) (width 0.25) (layer "F.Cu") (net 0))
 (segment (start 131.267278 71.60857) (end 131.684664 71.831668) (width 0.25) (layer "F.Cu") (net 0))
 (segment (start 112.884428 71.482924) (end 112.296406 71.55545) (width 0.25) (layer "F.Cu") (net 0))
 (segment (start 132.050506 72.131906) (end 141.4926 81.574) (width 0.25) (layer "F.Cu") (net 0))
 (segment (start 107.361273 73.45914) (end 106.876873 73.800294) (width 0.25) (layer "F.Cu") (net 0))
 (segment (start 110.000979 72.130424) (end 109.448202 72.343654) (width 0.25) (layer "F.Cu") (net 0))
 (segment (start 111.712651 71.656741) (end 111.134569 71.786554) (width 0.25) (layer "F.Cu") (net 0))
 (segment (start 141.4926 81.574) (end 141.4926 84.5092) (width 0.25) (layer "F.Cu") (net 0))
 (segment (start 130.814389 71.471188) (end 131.267278 71.60857) (width 0.25) (layer "F.Cu") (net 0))
 (segment (start 106.409795 74.164805) (end 105.961166 74.551795) (width 0.25) (layer "F.Cu") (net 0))
 (segment (start 108.377337 72.850135) (end 107.86183 73.142166) (width 0.25) (layer "F.Cu") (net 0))
 (segment (start 114.0676 71.4248) (end 113.4753 71.439339) (width 0.25) (layer "F.Cu") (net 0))
 (segment (start 108.906553 72.58375) (end 108.377337 72.850135) (width 0.25) (layer "F.Cu") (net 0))
 (segment (start 141.478 84.5058) (end 141.478 84.4946) (width 0.25) (layer "F.Cu") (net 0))
 (segment (start 113.4753 71.439339) (end 112.884428 71.482924) (width 0.25) (layer "F.Cu") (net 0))
 (segment (start 130.3434 71.4248) (end 114.0676 71.4248) (width 0.25) (layer "F.Cu") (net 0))
 (segment (start 109.448202 72.343654) (end 108.906553 72.58375) (width 0.25) (layer "F.Cu") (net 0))
 (segment (start 106.876873 73.800294) (end 106.409795 74.164805) (width 0.25) (layer "F.Cu") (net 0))
 (segment (start 105.532066 74.960333) (end 98.6028 81.8896) (width 0.25) (layer "F.Cu") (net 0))
 (segment (start 130.3434 71.4248) (end 130.814389 71.471188) (width 0.25) (layer "F.Cu") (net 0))
 (segment (start 111.134569 71.786554) (end 110.563553 71.944575) (width 0.25) (layer "F.Cu") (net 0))
 (segment (start 131.684664 71.831668) (end 132.050506 72.131906) (width 0.25) (layer "F.Cu") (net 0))
 (segment (start 112.296406 71.55545) (end 111.712651 71.656741) (width 0.25) (layer "F.Cu") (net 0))
 (segment (start 107.86183 73.142166) (end 107.361273 73.45914) (width 0.25) (layer "F.Cu") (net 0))
 (segment (start 105.961166 74.551795) (end 105.532066 74.960333) (width 0.25) (layer "F.Cu") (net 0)))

